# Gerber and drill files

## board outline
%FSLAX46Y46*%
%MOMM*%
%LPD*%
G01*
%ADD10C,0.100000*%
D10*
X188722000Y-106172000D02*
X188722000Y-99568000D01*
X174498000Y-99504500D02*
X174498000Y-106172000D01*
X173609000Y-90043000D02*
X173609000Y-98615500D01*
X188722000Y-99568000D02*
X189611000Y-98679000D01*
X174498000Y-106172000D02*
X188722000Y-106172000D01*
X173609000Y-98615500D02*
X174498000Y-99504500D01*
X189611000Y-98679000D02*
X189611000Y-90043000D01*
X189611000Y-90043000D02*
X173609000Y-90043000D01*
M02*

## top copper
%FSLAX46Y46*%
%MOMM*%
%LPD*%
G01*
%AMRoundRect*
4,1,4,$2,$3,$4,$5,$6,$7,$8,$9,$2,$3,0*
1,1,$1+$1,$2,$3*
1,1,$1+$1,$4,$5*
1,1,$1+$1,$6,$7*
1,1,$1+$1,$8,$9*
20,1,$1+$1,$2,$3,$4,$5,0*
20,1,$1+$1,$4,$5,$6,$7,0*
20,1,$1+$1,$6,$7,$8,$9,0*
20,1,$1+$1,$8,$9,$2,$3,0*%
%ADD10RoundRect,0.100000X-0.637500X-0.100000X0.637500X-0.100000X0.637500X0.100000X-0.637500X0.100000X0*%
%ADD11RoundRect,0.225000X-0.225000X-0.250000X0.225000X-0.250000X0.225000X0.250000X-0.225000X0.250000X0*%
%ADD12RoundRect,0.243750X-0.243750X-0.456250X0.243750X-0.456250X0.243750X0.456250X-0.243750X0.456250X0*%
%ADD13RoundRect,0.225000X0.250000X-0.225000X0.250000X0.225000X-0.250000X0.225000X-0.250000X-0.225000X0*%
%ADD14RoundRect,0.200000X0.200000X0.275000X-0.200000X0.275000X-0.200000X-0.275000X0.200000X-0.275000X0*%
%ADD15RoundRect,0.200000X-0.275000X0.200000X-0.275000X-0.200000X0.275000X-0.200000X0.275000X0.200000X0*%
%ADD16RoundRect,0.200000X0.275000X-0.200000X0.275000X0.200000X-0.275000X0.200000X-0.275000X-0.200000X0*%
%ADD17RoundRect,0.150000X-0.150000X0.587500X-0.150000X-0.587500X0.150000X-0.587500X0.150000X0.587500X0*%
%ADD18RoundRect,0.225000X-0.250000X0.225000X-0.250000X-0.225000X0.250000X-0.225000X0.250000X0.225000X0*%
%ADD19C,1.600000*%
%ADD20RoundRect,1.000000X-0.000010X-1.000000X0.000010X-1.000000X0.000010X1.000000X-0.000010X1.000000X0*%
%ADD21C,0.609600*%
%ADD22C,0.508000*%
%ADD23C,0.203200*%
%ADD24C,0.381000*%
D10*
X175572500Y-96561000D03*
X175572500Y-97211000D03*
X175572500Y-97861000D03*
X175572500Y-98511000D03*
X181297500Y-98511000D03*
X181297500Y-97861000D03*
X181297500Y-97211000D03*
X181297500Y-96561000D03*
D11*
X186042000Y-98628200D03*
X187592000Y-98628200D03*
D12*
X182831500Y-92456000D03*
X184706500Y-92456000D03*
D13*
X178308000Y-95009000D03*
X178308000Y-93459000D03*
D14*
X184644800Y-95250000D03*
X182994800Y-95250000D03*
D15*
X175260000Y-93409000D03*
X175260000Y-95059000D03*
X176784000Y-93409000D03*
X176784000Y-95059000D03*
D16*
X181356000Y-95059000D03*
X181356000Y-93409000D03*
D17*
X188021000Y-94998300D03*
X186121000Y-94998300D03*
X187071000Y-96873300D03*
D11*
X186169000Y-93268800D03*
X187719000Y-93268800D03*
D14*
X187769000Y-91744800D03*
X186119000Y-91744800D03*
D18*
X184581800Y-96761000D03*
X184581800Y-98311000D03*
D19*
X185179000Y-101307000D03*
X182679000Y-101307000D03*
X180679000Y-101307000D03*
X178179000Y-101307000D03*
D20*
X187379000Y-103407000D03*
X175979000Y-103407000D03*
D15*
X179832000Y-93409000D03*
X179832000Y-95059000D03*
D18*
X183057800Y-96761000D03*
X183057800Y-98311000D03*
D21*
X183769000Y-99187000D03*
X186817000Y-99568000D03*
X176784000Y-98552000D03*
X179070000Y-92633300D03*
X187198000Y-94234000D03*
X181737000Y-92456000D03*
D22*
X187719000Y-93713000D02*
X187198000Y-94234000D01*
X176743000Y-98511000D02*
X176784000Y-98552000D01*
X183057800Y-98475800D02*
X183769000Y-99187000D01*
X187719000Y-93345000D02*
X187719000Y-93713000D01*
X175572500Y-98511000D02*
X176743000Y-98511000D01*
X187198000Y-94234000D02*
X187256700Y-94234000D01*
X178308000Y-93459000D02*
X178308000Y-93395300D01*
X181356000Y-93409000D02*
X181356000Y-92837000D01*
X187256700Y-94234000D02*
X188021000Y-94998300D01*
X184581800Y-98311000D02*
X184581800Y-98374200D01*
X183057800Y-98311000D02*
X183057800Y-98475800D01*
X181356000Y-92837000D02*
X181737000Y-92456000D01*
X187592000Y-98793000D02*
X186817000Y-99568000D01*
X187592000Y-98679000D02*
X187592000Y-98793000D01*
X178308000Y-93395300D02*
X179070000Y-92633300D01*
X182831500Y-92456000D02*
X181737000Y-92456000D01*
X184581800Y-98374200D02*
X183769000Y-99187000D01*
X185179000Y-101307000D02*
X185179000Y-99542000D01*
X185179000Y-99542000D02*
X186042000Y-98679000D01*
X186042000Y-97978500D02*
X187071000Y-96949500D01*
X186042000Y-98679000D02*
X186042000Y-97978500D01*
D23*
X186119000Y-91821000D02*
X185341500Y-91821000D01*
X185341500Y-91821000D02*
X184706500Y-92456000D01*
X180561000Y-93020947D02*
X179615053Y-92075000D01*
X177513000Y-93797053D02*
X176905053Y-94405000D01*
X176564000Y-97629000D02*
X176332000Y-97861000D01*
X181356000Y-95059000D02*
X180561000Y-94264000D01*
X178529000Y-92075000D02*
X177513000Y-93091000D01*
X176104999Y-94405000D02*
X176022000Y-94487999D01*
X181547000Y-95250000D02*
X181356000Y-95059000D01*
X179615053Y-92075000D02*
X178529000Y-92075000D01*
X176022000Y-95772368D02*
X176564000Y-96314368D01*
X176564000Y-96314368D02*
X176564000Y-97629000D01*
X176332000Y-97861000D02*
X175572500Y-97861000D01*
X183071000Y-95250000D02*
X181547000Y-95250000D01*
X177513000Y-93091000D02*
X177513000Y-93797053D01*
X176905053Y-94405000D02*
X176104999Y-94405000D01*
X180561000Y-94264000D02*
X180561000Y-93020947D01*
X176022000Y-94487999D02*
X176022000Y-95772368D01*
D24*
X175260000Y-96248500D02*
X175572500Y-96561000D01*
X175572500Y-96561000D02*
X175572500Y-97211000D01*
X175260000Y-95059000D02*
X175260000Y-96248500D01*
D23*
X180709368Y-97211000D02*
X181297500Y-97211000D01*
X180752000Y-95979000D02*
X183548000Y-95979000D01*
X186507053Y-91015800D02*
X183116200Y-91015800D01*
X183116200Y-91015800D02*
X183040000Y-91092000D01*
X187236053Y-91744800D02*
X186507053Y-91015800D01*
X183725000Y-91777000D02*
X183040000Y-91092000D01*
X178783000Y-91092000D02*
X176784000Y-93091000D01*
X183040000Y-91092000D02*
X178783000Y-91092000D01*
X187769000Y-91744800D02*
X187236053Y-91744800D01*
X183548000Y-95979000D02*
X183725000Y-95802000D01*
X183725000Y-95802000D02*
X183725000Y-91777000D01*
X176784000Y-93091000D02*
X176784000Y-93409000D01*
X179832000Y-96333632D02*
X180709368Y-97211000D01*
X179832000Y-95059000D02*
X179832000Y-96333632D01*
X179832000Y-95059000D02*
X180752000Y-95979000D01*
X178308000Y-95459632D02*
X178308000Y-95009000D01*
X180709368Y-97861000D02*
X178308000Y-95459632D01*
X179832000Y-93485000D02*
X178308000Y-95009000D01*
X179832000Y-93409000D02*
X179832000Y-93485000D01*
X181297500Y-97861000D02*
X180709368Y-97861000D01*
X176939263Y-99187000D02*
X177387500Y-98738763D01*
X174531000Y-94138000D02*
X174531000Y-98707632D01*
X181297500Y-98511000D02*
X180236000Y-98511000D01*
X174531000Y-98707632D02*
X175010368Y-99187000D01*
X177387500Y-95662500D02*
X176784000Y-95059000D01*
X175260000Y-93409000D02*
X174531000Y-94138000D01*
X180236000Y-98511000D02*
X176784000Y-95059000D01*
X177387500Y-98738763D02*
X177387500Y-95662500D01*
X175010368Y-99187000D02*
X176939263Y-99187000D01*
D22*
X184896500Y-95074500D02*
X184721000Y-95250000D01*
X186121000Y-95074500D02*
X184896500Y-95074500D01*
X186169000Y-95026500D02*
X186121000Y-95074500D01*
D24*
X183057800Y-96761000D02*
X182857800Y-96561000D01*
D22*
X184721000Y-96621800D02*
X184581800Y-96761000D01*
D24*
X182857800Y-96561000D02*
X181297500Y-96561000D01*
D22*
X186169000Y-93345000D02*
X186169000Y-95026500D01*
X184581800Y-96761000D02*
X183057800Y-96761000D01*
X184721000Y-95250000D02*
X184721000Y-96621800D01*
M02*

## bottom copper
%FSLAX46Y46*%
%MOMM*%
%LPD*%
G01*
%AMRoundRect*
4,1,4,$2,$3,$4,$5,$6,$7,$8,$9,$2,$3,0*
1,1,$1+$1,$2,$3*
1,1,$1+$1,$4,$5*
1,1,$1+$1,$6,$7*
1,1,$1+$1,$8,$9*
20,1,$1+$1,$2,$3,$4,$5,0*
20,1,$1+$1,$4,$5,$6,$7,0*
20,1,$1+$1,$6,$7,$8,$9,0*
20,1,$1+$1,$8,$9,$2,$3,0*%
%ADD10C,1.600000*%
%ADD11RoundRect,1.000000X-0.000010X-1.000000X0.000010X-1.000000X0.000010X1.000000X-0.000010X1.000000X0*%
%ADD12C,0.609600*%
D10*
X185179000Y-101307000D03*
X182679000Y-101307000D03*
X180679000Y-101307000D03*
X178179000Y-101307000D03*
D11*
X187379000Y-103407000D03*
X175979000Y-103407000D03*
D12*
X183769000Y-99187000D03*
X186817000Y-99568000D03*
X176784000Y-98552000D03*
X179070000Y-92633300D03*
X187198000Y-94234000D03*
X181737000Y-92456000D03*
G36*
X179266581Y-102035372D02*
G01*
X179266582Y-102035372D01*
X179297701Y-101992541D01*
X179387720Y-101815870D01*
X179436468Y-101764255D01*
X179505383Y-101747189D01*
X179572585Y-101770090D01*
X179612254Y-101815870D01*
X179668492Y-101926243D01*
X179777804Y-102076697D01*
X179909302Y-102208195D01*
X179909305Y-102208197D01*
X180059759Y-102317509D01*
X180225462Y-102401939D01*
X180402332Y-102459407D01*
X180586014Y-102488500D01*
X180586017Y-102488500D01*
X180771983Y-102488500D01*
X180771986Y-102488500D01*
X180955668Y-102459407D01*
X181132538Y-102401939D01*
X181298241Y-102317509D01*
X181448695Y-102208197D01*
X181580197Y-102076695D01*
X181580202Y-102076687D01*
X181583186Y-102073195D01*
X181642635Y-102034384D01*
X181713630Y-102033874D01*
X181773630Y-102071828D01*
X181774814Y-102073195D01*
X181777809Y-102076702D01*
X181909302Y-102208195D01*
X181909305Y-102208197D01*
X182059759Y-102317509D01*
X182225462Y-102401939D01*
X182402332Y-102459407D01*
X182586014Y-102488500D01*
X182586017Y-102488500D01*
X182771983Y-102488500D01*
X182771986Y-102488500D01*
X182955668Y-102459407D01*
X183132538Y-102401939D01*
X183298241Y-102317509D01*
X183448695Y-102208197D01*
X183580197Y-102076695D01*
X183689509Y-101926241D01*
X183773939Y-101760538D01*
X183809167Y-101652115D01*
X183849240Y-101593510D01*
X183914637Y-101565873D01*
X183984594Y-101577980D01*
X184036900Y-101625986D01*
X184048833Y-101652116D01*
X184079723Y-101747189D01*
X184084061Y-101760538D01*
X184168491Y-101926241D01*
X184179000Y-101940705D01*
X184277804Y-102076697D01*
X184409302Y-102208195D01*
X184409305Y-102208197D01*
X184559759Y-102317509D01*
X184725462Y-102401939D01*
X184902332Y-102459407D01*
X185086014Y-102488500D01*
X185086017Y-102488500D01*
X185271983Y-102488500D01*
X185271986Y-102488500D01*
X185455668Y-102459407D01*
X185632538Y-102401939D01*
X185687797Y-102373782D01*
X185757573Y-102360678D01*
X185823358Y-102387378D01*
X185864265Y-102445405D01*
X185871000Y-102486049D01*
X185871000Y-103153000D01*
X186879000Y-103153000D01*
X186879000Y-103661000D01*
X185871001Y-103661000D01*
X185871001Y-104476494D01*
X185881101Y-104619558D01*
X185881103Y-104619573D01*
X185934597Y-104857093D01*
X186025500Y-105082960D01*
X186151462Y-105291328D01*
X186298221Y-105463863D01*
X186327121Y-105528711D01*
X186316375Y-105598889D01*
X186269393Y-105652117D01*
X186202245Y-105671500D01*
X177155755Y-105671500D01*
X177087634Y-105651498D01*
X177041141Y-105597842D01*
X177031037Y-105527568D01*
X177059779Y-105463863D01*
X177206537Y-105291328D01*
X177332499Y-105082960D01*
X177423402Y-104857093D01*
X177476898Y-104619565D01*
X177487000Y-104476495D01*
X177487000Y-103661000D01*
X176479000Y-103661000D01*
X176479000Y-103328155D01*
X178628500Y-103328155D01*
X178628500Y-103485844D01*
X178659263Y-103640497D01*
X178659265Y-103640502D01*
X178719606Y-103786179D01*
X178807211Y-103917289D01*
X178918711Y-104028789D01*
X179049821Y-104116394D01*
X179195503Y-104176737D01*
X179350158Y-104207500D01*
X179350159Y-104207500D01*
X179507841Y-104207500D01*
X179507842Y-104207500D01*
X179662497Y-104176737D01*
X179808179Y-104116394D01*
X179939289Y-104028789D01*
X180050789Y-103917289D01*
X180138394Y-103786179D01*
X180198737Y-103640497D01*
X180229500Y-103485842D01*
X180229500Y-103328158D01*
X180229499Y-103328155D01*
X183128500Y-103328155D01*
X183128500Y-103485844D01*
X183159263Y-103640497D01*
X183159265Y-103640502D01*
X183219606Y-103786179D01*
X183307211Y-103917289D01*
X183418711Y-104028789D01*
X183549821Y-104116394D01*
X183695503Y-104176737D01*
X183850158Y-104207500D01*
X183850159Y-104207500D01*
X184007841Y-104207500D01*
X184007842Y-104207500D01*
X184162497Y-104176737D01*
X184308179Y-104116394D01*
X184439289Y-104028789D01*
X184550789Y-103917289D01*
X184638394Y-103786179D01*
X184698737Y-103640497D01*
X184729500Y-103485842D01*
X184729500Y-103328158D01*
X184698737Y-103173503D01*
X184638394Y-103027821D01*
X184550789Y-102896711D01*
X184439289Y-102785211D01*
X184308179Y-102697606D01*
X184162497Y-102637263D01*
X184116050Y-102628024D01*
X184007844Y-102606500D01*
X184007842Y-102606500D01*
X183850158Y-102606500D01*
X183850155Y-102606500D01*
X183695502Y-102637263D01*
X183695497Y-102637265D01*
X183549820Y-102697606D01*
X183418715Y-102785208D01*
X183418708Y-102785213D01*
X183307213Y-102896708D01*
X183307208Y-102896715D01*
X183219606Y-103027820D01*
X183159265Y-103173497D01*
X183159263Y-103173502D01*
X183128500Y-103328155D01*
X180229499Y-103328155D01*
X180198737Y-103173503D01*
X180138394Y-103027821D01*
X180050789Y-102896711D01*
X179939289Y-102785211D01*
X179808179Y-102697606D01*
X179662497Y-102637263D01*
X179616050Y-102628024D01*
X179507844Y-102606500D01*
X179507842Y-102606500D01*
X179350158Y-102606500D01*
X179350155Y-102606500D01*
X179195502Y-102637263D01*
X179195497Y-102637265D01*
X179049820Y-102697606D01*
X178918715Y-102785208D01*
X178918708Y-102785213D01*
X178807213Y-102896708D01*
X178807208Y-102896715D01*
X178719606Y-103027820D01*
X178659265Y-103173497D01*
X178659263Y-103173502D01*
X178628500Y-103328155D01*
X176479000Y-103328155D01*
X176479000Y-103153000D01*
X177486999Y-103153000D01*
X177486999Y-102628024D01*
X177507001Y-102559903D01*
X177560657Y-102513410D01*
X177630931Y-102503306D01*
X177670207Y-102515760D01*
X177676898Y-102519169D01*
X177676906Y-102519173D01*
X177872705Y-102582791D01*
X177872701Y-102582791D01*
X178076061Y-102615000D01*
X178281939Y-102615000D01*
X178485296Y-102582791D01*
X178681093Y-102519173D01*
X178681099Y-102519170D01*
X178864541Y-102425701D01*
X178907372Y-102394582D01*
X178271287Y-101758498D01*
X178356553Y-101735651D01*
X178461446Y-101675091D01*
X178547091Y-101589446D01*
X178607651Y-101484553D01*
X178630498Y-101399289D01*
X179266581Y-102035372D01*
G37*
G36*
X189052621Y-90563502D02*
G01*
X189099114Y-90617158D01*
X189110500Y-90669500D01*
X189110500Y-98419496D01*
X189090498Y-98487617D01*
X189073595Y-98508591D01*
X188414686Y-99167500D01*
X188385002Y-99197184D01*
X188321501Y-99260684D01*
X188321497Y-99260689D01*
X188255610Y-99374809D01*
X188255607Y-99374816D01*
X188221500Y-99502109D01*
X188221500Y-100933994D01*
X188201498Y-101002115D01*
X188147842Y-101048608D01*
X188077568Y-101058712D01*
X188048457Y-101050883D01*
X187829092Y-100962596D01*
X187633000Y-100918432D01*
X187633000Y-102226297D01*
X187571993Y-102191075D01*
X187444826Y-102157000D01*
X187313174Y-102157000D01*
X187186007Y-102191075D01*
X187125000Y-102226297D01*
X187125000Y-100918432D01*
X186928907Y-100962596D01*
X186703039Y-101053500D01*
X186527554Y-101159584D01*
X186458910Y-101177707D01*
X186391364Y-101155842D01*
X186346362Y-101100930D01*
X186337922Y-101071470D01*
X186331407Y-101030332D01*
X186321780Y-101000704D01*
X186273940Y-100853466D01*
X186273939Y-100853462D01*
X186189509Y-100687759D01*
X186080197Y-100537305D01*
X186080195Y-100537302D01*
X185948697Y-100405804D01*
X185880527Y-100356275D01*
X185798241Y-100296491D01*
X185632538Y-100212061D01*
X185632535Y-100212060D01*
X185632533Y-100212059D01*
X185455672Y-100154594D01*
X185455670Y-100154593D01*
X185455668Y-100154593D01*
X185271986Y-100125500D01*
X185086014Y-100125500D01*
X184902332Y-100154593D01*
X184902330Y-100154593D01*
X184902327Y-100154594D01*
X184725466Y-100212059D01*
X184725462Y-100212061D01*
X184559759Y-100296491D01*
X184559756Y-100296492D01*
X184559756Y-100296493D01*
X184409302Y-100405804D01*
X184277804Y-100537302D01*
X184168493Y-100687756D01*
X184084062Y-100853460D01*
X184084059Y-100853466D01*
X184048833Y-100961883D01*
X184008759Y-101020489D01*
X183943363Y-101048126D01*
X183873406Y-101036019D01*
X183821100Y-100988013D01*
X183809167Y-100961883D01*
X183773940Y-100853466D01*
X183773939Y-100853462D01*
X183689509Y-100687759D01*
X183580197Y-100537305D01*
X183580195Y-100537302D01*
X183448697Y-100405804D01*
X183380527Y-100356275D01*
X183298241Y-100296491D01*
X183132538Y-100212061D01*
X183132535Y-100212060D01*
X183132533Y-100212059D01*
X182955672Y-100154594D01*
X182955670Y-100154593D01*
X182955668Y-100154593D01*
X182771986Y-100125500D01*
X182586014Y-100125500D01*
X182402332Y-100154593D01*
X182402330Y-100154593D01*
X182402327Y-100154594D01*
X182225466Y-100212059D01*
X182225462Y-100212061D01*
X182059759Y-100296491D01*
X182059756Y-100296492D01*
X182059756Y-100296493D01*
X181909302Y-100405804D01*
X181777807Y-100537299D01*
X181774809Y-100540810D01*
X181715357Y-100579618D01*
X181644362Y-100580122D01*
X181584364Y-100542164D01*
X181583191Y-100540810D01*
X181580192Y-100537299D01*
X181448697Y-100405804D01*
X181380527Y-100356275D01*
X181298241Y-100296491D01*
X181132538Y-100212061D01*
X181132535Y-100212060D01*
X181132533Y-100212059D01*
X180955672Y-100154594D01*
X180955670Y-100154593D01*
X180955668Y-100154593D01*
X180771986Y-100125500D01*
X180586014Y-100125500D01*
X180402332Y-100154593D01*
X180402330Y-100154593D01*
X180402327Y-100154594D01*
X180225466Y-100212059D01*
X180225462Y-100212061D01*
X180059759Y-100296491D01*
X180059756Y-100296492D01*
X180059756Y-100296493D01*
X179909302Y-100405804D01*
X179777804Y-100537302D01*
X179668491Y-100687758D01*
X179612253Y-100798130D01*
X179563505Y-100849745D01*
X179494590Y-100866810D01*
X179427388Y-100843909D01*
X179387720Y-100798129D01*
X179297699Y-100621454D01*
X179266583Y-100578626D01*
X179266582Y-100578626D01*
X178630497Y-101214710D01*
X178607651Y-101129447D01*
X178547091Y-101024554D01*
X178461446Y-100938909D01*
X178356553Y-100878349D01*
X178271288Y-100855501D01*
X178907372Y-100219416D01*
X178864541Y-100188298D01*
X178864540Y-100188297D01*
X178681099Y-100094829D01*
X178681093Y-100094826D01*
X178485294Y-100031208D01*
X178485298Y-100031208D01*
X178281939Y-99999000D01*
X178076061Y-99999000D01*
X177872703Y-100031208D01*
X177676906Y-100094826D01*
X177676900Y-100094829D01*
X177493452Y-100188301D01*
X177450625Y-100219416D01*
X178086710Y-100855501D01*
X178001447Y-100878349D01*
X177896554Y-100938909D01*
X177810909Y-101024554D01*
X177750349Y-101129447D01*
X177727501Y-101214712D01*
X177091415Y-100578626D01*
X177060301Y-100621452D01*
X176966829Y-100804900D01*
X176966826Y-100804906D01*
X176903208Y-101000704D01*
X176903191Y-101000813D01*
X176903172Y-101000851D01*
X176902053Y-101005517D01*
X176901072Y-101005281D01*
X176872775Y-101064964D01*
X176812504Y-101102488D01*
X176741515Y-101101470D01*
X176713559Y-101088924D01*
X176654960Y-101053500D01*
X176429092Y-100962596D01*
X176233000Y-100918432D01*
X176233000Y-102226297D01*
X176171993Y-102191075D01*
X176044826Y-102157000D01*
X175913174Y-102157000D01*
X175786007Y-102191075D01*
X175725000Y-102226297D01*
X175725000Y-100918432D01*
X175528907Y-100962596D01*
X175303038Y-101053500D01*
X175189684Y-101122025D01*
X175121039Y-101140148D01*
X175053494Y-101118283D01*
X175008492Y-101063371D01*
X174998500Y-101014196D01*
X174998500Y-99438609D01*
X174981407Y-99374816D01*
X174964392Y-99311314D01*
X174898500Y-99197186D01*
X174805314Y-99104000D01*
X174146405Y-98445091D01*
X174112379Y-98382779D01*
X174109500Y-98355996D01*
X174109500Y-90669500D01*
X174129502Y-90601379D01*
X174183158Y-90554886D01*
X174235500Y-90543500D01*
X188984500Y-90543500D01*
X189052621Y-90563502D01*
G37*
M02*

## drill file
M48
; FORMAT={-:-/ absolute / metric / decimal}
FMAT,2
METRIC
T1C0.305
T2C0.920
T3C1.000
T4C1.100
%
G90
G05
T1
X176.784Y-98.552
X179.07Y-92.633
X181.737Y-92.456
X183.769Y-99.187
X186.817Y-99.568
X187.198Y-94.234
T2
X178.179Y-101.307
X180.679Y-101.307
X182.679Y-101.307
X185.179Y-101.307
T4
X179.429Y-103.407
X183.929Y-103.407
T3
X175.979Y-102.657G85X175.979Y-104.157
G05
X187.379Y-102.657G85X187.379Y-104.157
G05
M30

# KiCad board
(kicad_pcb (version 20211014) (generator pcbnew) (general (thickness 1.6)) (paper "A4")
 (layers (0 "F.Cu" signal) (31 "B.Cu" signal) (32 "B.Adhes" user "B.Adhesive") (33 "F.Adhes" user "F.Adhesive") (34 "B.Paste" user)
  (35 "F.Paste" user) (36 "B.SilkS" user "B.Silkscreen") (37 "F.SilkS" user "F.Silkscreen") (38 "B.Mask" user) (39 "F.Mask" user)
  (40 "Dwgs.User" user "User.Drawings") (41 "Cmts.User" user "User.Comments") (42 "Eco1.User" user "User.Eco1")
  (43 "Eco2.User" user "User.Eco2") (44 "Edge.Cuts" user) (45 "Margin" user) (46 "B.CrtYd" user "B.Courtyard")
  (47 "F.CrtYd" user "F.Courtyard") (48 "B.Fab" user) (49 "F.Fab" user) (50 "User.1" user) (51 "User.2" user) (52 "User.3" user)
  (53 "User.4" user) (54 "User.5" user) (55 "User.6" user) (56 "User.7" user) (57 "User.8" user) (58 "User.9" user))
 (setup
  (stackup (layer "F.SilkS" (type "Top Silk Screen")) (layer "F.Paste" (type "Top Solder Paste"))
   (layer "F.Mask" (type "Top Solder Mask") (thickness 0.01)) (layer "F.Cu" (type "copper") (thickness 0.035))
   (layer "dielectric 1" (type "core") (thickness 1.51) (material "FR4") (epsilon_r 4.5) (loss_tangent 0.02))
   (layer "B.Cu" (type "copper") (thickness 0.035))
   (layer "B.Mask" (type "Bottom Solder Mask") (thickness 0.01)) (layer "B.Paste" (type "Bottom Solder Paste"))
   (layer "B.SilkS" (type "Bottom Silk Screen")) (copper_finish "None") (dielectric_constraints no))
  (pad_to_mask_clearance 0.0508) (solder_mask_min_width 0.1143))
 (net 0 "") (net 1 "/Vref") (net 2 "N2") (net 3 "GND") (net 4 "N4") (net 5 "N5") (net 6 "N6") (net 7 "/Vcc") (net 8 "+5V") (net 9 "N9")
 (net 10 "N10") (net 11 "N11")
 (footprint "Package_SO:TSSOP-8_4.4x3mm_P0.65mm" (layer "F.Cu") (at 178.435 97.536)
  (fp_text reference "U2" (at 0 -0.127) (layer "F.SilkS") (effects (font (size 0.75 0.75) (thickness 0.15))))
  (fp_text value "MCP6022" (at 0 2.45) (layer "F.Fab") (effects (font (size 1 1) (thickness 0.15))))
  (pad "1" smd roundrect (at -2.8625 -0.975) (size 1.475 0.4) (layers "F.Cu" "F.Paste" "F.Mask") (roundrect_rratio 0.25) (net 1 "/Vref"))
  (pad "2" smd roundrect (at -2.8625 -0.325) (size 1.475 0.4) (layers "F.Cu" "F.Paste" "F.Mask") (roundrect_rratio 0.25) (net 1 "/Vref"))
  (pad "3" smd roundrect (at -2.8625 0.325) (size 1.475 0.4) (layers "F.Cu" "F.Paste" "F.Mask") (roundrect_rratio 0.25) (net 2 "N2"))
  (pad "4" smd roundrect (at -2.8625 0.975) (size 1.475 0.4) (layers "F.Cu" "F.Paste" "F.Mask") (roundrect_rratio 0.25) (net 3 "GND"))
  (pad "5" smd roundrect (at 2.8625 0.975) (size 1.475 0.4) (layers "F.Cu" "F.Paste" "F.Mask") (roundrect_rratio 0.25) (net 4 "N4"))
  (pad "6" smd roundrect (at 2.8625 0.325) (size 1.475 0.4) (layers "F.Cu" "F.Paste" "F.Mask") (roundrect_rratio 0.25) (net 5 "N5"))
  (pad "7" smd roundrect (at 2.8625 -0.325) (size 1.475 0.4) (layers "F.Cu" "F.Paste" "F.Mask") (roundrect_rratio 0.25) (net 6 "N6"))
  (pad "8" smd roundrect (at 2.8625 -0.975) (size 1.475 0.4) (layers "F.Cu" "F.Paste" "F.Mask") (roundrect_rratio 0.25) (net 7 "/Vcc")))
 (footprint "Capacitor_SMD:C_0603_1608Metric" (layer "F.Cu") (at 186.817 98.6282)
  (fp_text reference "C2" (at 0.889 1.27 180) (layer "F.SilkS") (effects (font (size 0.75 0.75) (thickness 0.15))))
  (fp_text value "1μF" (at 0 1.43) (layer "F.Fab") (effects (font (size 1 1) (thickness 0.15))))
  (pad "1" smd roundrect (at -0.775 0) (size 0.9 0.95) (layers "F.Cu" "F.Paste" "F.Mask") (roundrect_rratio 0.25) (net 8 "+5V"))
  (pad "2" smd roundrect (at 0.775 0) (size 0.9 0.95) (layers "F.Cu" "F.Paste" "F.Mask") (roundrect_rratio 0.25) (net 3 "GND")))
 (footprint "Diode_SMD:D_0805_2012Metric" (layer "F.Cu") (at 183.769 92.456)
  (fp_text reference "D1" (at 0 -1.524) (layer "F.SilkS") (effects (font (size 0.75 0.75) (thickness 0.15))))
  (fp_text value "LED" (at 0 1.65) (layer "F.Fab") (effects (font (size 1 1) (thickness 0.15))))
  (pad "1" smd roundrect (at -0.9375 0) (size 0.975 1.4) (layers "F.Cu" "F.Paste" "F.Mask") (roundrect_rratio 0.25) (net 3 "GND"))
  (pad "2" smd roundrect (at 0.9375 0) (size 0.975 1.4) (layers "F.Cu" "F.Paste" "F.Mask") (roundrect_rratio 0.25) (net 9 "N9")))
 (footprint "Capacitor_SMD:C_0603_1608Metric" (layer "F.Cu") (at 178.308 94.234 90)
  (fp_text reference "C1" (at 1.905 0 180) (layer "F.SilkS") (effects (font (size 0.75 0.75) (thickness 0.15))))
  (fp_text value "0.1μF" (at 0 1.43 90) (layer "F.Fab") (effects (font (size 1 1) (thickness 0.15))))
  (pad "1" smd roundrect (at -0.775 0 90) (size 0.9 0.95) (layers "F.Cu" "F.Paste" "F.Mask") (roundrect_rratio 0.25) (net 5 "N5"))
  (pad "2" smd roundrect (at 0.775 0 90) (size 0.9 0.95) (layers "F.Cu" "F.Paste" "F.Mask") (roundrect_rratio 0.25) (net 3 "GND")))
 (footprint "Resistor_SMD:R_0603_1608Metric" (layer "F.Cu") (at 183.8198 95.25 180)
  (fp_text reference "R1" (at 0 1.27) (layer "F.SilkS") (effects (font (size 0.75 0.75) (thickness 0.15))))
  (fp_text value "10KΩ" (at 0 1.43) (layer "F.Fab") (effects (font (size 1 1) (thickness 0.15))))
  (pad "1" smd roundrect (at -0.825 0 180) (size 0.8 0.95) (layers "F.Cu" "F.Paste" "F.Mask") (roundrect_rratio 0.25) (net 7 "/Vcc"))
  (pad "2" smd roundrect (at 0.825 0 180) (size 0.8 0.95) (layers "F.Cu" "F.Paste" "F.Mask") (roundrect_rratio 0.25) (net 2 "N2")))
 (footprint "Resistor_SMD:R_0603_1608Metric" (layer "F.Cu") (at 175.26 94.234 -90)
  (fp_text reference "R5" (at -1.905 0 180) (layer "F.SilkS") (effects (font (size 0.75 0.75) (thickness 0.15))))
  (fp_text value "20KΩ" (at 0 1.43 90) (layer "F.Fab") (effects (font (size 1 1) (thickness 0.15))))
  (pad "1" smd roundrect (at -0.825 0 270) (size 0.8 0.95) (layers "F.Cu" "F.Paste" "F.Mask") (roundrect_rratio 0.25) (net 4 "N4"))
  (pad "2" smd roundrect (at 0.825 0 270) (size 0.8 0.95) (layers "F.Cu" "F.Paste" "F.Mask") (roundrect_rratio 0.25) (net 1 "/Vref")))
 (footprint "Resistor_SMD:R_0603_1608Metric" (layer "F.Cu") (at 176.784 94.234 -90)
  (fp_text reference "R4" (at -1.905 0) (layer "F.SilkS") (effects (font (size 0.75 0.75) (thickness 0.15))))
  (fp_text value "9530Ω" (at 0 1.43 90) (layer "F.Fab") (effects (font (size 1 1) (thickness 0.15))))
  (pad "1" smd roundrect (at -0.825 0 270) (size 0.8 0.95) (layers "F.Cu" "F.Paste" "F.Mask") (roundrect_rratio 0.25) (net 6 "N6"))
  (pad "2" smd roundrect (at 0.825 0 270) (size 0.8 0.95) (layers "F.Cu" "F.Paste" "F.Mask") (roundrect_rratio 0.25) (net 4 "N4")))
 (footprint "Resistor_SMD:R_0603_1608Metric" (layer "F.Cu") (at 181.356 94.234 90)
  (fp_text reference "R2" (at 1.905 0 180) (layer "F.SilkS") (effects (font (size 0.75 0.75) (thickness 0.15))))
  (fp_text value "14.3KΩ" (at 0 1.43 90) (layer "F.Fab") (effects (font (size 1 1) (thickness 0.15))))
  (pad "1" smd roundrect (at -0.825 0 90) (size 0.8 0.95) (layers "F.Cu" "F.Paste" "F.Mask") (roundrect_rratio 0.25) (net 2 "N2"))
  (pad "2" smd roundrect (at 0.825 0 90) (size 0.8 0.95) (layers "F.Cu" "F.Paste" "F.Mask") (roundrect_rratio 0.25) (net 3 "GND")))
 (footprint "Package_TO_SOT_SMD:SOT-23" (layer "F.Cu") (at 187.071 95.9358 -90)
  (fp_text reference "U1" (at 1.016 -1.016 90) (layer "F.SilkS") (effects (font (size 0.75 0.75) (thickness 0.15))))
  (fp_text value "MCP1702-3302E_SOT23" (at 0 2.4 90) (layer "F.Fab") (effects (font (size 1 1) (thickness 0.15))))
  (pad "1" smd roundrect (at -0.9375 -0.95 270) (size 1.475 0.6) (layers "F.Cu" "F.Paste" "F.Mask") (roundrect_rratio 0.25) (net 3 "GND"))
  (pad "2" smd roundrect (at -0.9375 0.95 270) (size 1.475 0.6) (layers "F.Cu" "F.Paste" "F.Mask") (roundrect_rratio 0.25) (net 7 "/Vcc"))
  (pad "3" smd roundrect (at 0.9375 0 270) (size 1.475 0.6) (layers "F.Cu" "F.Paste" "F.Mask") (roundrect_rratio 0.25) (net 8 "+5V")))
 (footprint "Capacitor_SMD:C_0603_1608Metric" (layer "F.Cu") (at 186.944 93.2688)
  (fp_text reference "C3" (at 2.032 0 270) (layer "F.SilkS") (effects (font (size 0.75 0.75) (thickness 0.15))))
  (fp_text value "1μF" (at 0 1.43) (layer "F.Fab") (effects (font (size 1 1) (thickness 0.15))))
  (pad "1" smd roundrect (at -0.775 0) (size 0.9 0.95) (layers "F.Cu" "F.Paste" "F.Mask") (roundrect_rratio 0.25) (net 7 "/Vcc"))
  (pad "2" smd roundrect (at 0.775 0) (size 0.9 0.95) (layers "F.Cu" "F.Paste" "F.Mask") (roundrect_rratio 0.25) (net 3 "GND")))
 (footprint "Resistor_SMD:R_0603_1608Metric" (layer "F.Cu") (at 186.944 91.7448 180)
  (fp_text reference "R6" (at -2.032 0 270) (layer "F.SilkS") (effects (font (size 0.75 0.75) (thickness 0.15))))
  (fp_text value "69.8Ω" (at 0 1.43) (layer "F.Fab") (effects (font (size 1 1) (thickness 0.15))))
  (pad "1" smd roundrect (at -0.825 0 180) (size 0.8 0.95) (layers "F.Cu" "F.Paste" "F.Mask") (roundrect_rratio 0.25) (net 6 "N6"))
  (pad "2" smd roundrect (at 0.825 0 180) (size 0.8 0.95) (layers "F.Cu" "F.Paste" "F.Mask") (roundrect_rratio 0.25) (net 9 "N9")))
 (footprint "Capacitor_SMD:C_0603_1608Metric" (layer "F.Cu") (at 184.5818 97.536 -90)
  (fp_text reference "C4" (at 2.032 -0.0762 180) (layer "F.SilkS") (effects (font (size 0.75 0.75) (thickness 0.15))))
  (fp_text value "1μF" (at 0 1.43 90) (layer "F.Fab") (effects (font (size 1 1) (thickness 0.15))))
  (pad "1" smd roundrect (at -0.775 0 270) (size 0.9 0.95) (layers "F.Cu" "F.Paste" "F.Mask") (roundrect_rratio 0.25) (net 7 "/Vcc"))
  (pad "2" smd roundrect (at 0.775 0 270) (size 0.9 0.95) (layers "F.Cu" "F.Paste" "F.Mask") (roundrect_rratio 0.25) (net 3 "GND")))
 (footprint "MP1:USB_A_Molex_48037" (layer "F.Cu") (at 181.679 103.407)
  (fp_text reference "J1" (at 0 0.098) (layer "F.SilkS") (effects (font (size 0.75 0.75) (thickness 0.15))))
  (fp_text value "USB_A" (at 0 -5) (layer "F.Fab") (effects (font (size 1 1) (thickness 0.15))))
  (pad "" np_thru_hole circle (at 2.25 0) (size 1.1 1.1) (drill 1.1) (layers F&B.Cu *.Mask))
  (pad "" np_thru_hole circle (at -2.25 0) (size 1.1 1.1) (drill 1.1) (layers F&B.Cu *.Mask))
  (pad "1" thru_hole circle (at 3.5 -2.1) (size 1.6 1.6) (drill 0.92) (layers *.Cu *.Mask) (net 8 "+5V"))
  (pad "2" thru_hole circle (at 1 -2.1) (size 1.6 1.6) (drill 0.92) (layers *.Cu *.Mask) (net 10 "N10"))
  (pad "3" thru_hole circle (at -1 -2.1) (size 1.6 1.6) (drill 0.92) (layers *.Cu *.Mask) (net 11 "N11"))
  (pad "4" thru_hole circle (at -3.5 -2.1) (size 1.6 1.6) (drill 0.92) (layers *.Cu *.Mask) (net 3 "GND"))
  (pad "5" thru_hole roundrect (at 5.7 0) (size 2 4) (drill oval 1 2.5) (layers *.Cu *.Mask) (roundrect_rratio 0.5) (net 3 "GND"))
  (pad "5" thru_hole roundrect (at -5.7 0) (size 2 4) (drill oval 1 2.5) (layers *.Cu *.Mask) (roundrect_rratio 0.5) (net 3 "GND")))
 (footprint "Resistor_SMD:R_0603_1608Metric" (layer "F.Cu") (at 179.832 94.234 -90)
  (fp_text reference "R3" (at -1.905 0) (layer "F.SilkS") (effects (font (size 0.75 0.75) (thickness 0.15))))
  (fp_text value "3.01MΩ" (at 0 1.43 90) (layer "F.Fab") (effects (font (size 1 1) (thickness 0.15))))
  (pad "1" smd roundrect (at -0.825 0 270) (size 0.8 0.95) (layers "F.Cu" "F.Paste" "F.Mask") (roundrect_rratio 0.25) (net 5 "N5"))
  (pad "2" smd roundrect (at 0.825 0 270) (size 0.8 0.95) (layers "F.Cu" "F.Paste" "F.Mask") (roundrect_rratio 0.25) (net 6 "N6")))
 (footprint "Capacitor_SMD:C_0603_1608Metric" (layer "F.Cu") (at 183.0578 97.536 -90)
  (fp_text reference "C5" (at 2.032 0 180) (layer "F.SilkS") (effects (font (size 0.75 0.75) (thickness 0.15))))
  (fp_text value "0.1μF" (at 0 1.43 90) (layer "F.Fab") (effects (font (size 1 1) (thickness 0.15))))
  (pad "1" smd roundrect (at -0.775 0 270) (size 0.9 0.95) (layers "F.Cu" "F.Paste" "F.Mask") (roundrect_rratio 0.25) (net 7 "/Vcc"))
  (pad "2" smd roundrect (at 0.775 0 270) (size 0.9 0.95) (layers "F.Cu" "F.Paste" "F.Mask") (roundrect_rratio 0.25) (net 3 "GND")))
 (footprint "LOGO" (layer "B.Cu") (at 178.308 94.615 90)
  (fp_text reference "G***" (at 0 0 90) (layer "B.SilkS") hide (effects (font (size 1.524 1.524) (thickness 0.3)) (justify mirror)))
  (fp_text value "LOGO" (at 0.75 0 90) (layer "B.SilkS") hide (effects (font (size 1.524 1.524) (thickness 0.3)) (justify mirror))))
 (gr_line (start 188.722 106.172) (end 188.722 99.568) (layer "Edge.Cuts") (width 0.1))
 (gr_line (start 174.498 99.5045) (end 174.498 106.172) (layer "Edge.Cuts") (width 0.1))
 (gr_line (start 173.609 90.043) (end 173.609 98.6155) (layer "Edge.Cuts") (width 0.1))
 (gr_line (start 188.722 99.568) (end 189.611 98.679) (layer "Edge.Cuts") (width 0.1))
 (gr_line (start 174.498 106.172) (end 188.722 106.172) (layer "Edge.Cuts") (width 0.1))
 (gr_line (start 173.609 98.6155) (end 174.498 99.5045) (layer "Edge.Cuts") (width 0.1))
 (gr_line (start 189.611 98.679) (end 189.611 90.043) (layer "Edge.Cuts") (width 0.1))
 (gr_line (start 189.611 90.043) (end 173.609 90.043) (layer "Edge.Cuts") (width 0.1))
 (segment (start 187.719 93.713) (end 187.198 94.234) (width 0.508) (layer "F.Cu") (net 3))
 (segment (start 176.743 98.511) (end 176.784 98.552) (width 0.508) (layer "F.Cu") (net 3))
 (segment (start 183.0578 98.4758) (end 183.769 99.187) (width 0.508) (layer "F.Cu") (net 3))
 (segment (start 187.719 93.345) (end 187.719 93.713) (width 0.508) (layer "F.Cu") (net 3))
 (segment (start 175.5725 98.511) (end 176.743 98.511) (width 0.508) (layer "F.Cu") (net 3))
 (segment (start 187.198 94.234) (end 187.2567 94.234) (width 0.508) (layer "F.Cu") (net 3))
 (segment (start 178.308 93.459) (end 178.308 93.3953) (width 0.508) (layer "F.Cu") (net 3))
 (segment (start 181.356 93.409) (end 181.356 92.837) (width 0.508) (layer "F.Cu") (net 3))
 (segment (start 187.2567 94.234) (end 188.021 94.9983) (width 0.508) (layer "F.Cu") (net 3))
 (segment (start 184.5818 98.311) (end 184.5818 98.3742) (width 0.508) (layer "F.Cu") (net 3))
 (segment (start 183.0578 98.311) (end 183.0578 98.4758) (width 0.508) (layer "F.Cu") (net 3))
 (segment (start 181.356 92.837) (end 181.737 92.456) (width 0.508) (layer "F.Cu") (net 3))
 (segment (start 187.592 98.793) (end 186.817 99.568) (width 0.508) (layer "F.Cu") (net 3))
 (segment (start 187.592 98.679) (end 187.592 98.793) (width 0.508) (layer "F.Cu") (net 3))
 (segment (start 178.308 93.3953) (end 179.07 92.6333) (width 0.508) (layer "F.Cu") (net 3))
 (segment (start 182.8315 92.456) (end 181.737 92.456) (width 0.508) (layer "F.Cu") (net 3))
 (segment (start 184.5818 98.3742) (end 183.769 99.187) (width 0.508) (layer "F.Cu") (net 3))
 (via (at 183.769 99.187) (size 0.6096) (drill 0.3048) (layers "F.Cu" "B.Cu") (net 3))
 (via (at 186.817 99.568) (size 0.6096) (drill 0.3048) (layers "F.Cu" "B.Cu") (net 3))
 (via (at 176.784 98.552) (size 0.6096) (drill 0.3048) (layers "F.Cu" "B.Cu") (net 3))
 (via (at 179.07 92.6333) (size 0.6096) (drill 0.3048) (layers "F.Cu" "B.Cu") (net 3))
 (via (at 187.198 94.234) (size 0.6096) (drill 0.3048) (layers "F.Cu" "B.Cu") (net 3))
 (via (at 181.737 92.456) (size 0.6096) (drill 0.3048) (layers "F.Cu" "B.Cu") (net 3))
 (segment (start 185.179 101.307) (end 185.179 99.542) (width 0.508) (layer "F.Cu") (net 8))
 (segment (start 185.179 99.542) (end 186.042 98.679) (width 0.508) (layer "F.Cu") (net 8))
 (segment (start 186.042 97.9785) (end 187.071 96.9495) (width 0.508) (layer "F.Cu") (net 8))
 (segment (start 186.042 98.679) (end 186.042 97.9785) (width 0.508) (layer "F.Cu") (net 8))
 (segment (start 186.119 91.821) (end 185.3415 91.821) (width 0.2032) (layer "F.Cu") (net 9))
 (segment (start 185.3415 91.821) (end 184.7065 92.456) (width 0.2032) (layer "F.Cu") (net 9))
 (segment (start 180.561 93.020947) (end 179.615053 92.075) (width 0.2032) (layer "F.Cu") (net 2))
 (segment (start 177.513 93.797053) (end 176.905053 94.405) (width 0.2032) (layer "F.Cu") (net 2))
 (segment (start 176.564 97.629) (end 176.332 97.861) (width 0.2032) (layer "F.Cu") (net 2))
 (segment (start 181.356 95.059) (end 180.561 94.264) (width 0.2032) (layer "F.Cu") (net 2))
 (segment (start 178.529 92.075) (end 177.513 93.091) (width 0.2032) (layer "F.Cu") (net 2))
 (segment (start 176.104999 94.405) (end 176.022 94.487999) (width 0.2032) (layer "F.Cu") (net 2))
 (segment (start 181.547 95.25) (end 181.356 95.059) (width 0.2032) (layer "F.Cu") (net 2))
 (segment (start 179.615053 92.075) (end 178.529 92.075) (width 0.2032) (layer "F.Cu") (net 2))
 (segment (start 176.022 95.772368) (end 176.564 96.314368) (width 0.2032) (layer "F.Cu") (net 2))
 (segment (start 176.564 96.314368) (end 176.564 97.629) (width 0.2032) (layer "F.Cu") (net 2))
 (segment (start 176.332 97.861) (end 175.5725 97.861) (width 0.2032) (layer "F.Cu") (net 2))
 (segment (start 183.071 95.25) (end 181.547 95.25) (width 0.2032) (layer "F.Cu") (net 2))
 (segment (start 177.513 93.091) (end 177.513 93.797053) (width 0.2032) (layer "F.Cu") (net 2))
 (segment (start 176.905053 94.405) (end 176.104999 94.405) (width 0.2032) (layer "F.Cu") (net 2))
 (segment (start 180.561 94.264) (end 180.561 93.020947) (width 0.2032) (layer "F.Cu") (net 2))
 (segment (start 176.022 94.487999) (end 176.022 95.772368) (width 0.2032) (layer "F.Cu") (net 2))
 (segment (start 175.26 96.2485) (end 175.5725 96.561) (width 0.381) (layer "F.Cu") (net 1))
 (segment (start 175.5725 96.561) (end 175.5725 97.211) (width 0.381) (layer "F.Cu") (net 1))
 (segment (start 175.26 95.059) (end 175.26 96.2485) (width 0.381) (layer "F.Cu") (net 1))
 (segment (start 180.709368 97.211) (end 181.2975 97.211) (width 0.2032) (layer "F.Cu") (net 6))
 (segment (start 180.752 95.979) (end 183.548 95.979) (width 0.2032) (layer "F.Cu") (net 6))
 (segment (start 186.507053 91.0158) (end 183.1162 91.0158) (width 0.2032) (layer "F.Cu") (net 6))
 (segment (start 183.1162 91.0158) (end 183.04 91.092) (width 0.2032) (layer "F.Cu") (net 6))
 (segment (start 187.236053 91.7448) (end 186.507053 91.0158) (width 0.2032) (layer "F.Cu") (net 6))
 (segment (start 183.725 91.777) (end 183.04 91.092) (width 0.2032) (layer "F.Cu") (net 6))
 (segment (start 178.783 91.092) (end 176.784 93.091) (width 0.2032) (layer "F.Cu") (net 6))
 (segment (start 183.04 91.092) (end 178.783 91.092) (width 0.2032) (layer "F.Cu") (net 6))
 (segment (start 187.769 91.7448) (end 187.236053 91.7448) (width 0.2032) (layer "F.Cu") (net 6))
 (segment (start 183.548 95.979) (end 183.725 95.802) (width 0.2032) (layer "F.Cu") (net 6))
 (segment (start 183.725 95.802) (end 183.725 91.777) (width 0.2032) (layer "F.Cu") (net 6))
 (segment (start 176.784 93.091) (end 176.784 93.409) (width 0.2032) (layer "F.Cu") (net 6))
 (segment (start 179.832 96.333632) (end 180.709368 97.211) (width 0.2032) (layer "F.Cu") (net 6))
 (segment (start 179.832 95.059) (end 179.832 96.333632) (width 0.2032) (layer "F.Cu") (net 6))
 (segment (start 179.832 95.059) (end 180.752 95.979) (width 0.2032) (layer "F.Cu") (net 6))
 (segment (start 178.308 95.459632) (end 178.308 95.009) (width 0.2032) (layer "F.Cu") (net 5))
 (segment (start 180.709368 97.861) (end 178.308 95.459632) (width 0.2032) (layer "F.Cu") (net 5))
 (segment (start 179.832 93.485) (end 178.308 95.009) (width 0.2032) (layer "F.Cu") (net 5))
 (segment (start 179.832 93.409) (end 179.832 93.485) (width 0.2032) (layer "F.Cu") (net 5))
 (segment (start 181.2975 97.861) (end 180.709368 97.861) (width 0.2032) (layer "F.Cu") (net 5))
 (segment (start 176.939263 99.187) (end 177.3875 98.738763) (width 0.2032) (layer "F.Cu") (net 4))
 (segment (start 174.531 94.138) (end 174.531 98.707632) (width 0.2032) (layer "F.Cu") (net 4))
 (segment (start 181.2975 98.511) (end 180.236 98.511) (width 0.2032) (layer "F.Cu") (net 4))
 (segment (start 174.531 98.707632) (end 175.010368 99.187) (width 0.2032) (layer "F.Cu") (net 4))
 (segment (start 177.3875 95.6625) (end 176.784 95.059) (width 0.2032) (layer "F.Cu") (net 4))
 (segment (start 175.26 93.409) (end 174.531 94.138) (width 0.2032) (layer "F.Cu") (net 4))
 (segment (start 180.236 98.511) (end 176.784 95.059) (width 0.2032) (layer "F.Cu") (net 4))
 (segment (start 177.3875 98.738763) (end 177.3875 95.6625) (width 0.2032) (layer "F.Cu") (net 4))
 (segment (start 175.010368 99.187) (end 176.939263 99.187) (width 0.2032) (layer "F.Cu") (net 4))
 (segment (start 184.8965 95.0745) (end 184.721 95.25) (width 0.508) (layer "F.Cu") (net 7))
 (segment (start 186.121 95.0745) (end 184.8965 95.0745) (width 0.508) (layer "F.Cu") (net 7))
 (segment (start 186.169 95.0265) (end 186.121 95.0745) (width 0.508) (layer "F.Cu") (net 7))
 (segment (start 183.0578 96.761) (end 182.8578 96.561) (width 0.381) (layer "F.Cu") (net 7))
 (segment (start 184.721 96.6218) (end 184.5818 96.761) (width 0.508) (layer "F.Cu") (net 7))
 (segment (start 182.8578 96.561) (end 181.2975 96.561) (width 0.381) (layer "F.Cu") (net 7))
 (segment (start 186.169 93.345) (end 186.169 95.0265) (width 0.508) (layer "F.Cu") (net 7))
 (segment (start 184.5818 96.761) (end 183.0578 96.761) (width 0.508) (layer "F.Cu") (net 7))
 (segment (start 184.721 95.25) (end 184.721 96.6218) (width 0.508) (layer "F.Cu") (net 7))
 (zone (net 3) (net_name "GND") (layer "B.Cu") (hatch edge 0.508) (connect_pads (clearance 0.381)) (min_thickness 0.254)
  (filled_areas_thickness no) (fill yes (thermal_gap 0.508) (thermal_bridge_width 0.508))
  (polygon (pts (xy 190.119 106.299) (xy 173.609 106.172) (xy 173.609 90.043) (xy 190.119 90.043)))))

